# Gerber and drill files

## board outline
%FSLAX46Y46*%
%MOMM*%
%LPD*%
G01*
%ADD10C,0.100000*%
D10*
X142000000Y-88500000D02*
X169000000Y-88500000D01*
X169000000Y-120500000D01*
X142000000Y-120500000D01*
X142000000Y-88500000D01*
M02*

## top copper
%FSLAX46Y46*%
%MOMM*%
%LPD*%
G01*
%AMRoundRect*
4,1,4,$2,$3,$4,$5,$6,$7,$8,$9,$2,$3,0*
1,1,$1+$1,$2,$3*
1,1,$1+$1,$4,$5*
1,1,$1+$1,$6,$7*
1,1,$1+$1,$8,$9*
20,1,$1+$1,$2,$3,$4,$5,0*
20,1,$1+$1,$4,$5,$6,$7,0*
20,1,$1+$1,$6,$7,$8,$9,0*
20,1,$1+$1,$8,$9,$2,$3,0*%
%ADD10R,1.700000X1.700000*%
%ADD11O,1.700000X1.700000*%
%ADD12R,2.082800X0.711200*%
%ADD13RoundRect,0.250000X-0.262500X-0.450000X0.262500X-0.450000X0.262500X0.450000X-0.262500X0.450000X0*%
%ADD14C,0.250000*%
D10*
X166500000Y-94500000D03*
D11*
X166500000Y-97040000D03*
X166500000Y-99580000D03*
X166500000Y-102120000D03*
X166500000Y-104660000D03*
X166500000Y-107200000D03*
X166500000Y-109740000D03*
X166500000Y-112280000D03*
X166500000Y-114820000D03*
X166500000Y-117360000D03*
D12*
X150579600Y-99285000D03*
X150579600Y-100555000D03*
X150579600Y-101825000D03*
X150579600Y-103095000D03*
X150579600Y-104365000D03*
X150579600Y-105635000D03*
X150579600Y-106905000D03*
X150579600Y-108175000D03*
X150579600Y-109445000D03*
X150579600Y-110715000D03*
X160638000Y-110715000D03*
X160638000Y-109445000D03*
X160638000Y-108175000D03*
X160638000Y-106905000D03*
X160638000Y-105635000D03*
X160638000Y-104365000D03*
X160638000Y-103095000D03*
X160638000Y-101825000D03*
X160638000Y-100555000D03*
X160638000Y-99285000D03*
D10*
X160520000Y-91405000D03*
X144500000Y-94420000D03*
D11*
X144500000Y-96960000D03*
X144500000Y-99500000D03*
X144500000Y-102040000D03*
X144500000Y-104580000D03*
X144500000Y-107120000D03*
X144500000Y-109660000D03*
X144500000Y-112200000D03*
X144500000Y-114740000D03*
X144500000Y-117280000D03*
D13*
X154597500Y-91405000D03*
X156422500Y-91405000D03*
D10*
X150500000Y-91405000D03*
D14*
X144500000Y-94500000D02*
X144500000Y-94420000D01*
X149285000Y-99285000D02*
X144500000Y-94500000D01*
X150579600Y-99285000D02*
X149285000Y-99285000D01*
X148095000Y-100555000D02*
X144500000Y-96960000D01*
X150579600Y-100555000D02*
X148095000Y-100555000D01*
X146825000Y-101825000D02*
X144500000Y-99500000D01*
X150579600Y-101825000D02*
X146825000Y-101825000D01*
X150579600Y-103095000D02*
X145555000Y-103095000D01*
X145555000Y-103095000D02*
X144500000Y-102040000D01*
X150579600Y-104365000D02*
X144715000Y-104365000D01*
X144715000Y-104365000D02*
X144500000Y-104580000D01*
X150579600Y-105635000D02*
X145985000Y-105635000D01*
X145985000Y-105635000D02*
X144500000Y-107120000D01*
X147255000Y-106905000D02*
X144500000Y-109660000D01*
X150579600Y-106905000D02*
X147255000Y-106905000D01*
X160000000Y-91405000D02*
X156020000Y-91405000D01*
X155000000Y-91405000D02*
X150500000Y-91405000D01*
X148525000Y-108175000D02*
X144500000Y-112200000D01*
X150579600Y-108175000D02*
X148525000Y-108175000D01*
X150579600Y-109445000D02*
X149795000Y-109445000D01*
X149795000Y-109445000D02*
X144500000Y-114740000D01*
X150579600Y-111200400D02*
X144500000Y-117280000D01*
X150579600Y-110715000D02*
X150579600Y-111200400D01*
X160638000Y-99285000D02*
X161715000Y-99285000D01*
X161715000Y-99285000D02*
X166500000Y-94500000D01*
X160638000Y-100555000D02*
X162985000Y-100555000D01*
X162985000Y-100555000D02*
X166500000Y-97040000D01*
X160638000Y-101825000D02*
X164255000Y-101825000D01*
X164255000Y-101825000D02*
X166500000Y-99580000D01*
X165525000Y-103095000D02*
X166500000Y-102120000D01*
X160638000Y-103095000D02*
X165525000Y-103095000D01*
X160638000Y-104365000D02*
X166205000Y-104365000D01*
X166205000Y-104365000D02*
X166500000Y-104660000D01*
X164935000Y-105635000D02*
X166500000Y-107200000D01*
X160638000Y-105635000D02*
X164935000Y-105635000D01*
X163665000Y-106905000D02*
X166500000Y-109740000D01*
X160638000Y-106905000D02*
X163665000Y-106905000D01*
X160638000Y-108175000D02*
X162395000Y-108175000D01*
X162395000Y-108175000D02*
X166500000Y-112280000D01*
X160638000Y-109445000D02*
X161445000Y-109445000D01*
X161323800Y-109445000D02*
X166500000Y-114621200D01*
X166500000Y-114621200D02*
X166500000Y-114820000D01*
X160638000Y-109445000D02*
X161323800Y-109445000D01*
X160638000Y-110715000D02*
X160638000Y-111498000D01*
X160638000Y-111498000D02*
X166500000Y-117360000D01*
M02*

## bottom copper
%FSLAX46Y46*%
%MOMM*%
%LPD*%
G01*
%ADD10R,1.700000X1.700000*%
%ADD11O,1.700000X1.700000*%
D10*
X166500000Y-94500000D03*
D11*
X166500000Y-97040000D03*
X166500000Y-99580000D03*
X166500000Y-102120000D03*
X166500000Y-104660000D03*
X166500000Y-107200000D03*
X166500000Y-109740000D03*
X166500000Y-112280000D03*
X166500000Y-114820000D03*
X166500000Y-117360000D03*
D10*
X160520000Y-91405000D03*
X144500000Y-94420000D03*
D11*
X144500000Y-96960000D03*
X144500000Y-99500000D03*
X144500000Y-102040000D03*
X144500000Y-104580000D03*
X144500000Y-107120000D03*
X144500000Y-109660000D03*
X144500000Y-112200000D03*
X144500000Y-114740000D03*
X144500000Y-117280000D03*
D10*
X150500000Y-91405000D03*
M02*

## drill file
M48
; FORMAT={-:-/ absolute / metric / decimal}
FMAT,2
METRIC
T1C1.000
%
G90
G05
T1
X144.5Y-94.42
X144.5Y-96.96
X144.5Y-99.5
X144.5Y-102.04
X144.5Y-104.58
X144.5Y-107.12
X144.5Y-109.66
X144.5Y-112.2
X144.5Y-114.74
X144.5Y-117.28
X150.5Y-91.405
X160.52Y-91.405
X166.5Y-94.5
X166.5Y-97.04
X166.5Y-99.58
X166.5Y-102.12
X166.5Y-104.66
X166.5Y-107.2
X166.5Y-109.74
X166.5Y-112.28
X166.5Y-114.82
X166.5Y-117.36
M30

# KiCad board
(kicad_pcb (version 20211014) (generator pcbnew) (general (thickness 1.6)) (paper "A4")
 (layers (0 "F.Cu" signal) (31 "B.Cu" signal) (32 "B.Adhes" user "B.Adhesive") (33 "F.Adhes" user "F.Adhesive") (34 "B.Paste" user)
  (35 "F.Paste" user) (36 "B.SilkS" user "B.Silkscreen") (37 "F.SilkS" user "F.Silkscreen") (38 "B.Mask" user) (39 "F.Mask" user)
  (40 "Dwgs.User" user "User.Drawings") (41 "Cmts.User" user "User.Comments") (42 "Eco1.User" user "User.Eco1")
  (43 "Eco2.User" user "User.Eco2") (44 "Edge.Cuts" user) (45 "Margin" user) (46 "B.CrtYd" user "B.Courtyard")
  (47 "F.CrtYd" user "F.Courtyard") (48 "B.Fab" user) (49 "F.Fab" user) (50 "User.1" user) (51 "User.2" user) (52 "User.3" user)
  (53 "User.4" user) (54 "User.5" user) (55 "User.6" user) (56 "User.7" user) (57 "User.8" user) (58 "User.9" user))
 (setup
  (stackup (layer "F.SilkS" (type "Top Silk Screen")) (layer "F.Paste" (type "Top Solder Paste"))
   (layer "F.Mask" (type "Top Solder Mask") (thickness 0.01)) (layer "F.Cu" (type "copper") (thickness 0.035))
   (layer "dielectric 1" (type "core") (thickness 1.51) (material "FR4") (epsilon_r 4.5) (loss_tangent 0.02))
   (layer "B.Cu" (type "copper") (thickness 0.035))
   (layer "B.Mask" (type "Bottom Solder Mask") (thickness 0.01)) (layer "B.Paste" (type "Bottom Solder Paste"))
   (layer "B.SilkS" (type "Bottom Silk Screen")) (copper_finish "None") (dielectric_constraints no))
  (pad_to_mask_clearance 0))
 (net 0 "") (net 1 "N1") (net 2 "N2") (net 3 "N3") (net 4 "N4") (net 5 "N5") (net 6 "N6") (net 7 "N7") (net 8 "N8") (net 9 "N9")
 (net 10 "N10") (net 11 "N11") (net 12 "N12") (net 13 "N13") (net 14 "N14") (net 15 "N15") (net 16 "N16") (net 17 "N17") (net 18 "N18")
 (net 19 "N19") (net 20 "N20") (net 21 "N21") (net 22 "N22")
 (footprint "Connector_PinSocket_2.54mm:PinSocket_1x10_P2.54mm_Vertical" (layer "F.Cu") (at 166.5 94.5)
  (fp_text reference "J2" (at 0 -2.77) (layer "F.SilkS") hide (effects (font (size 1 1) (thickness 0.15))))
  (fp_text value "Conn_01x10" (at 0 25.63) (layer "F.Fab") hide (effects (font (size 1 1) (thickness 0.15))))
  (pad "1" thru_hole rect (at 0 0) (size 1.7 1.7) (drill 1) (layers *.Cu *.Mask) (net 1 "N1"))
  (pad "2" thru_hole oval (at 0 2.54) (size 1.7 1.7) (drill 1) (layers *.Cu *.Mask) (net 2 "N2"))
  (pad "3" thru_hole oval (at 0 5.08) (size 1.7 1.7) (drill 1) (layers *.Cu *.Mask) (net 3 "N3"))
  (pad "4" thru_hole oval (at 0 7.62) (size 1.7 1.7) (drill 1) (layers *.Cu *.Mask) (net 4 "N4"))
  (pad "5" thru_hole oval (at 0 10.16) (size 1.7 1.7) (drill 1) (layers *.Cu *.Mask) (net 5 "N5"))
  (pad "6" thru_hole oval (at 0 12.7) (size 1.7 1.7) (drill 1) (layers *.Cu *.Mask) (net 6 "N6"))
  (pad "7" thru_hole oval (at 0 15.24) (size 1.7 1.7) (drill 1) (layers *.Cu *.Mask) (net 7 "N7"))
  (pad "8" thru_hole oval (at 0 17.78) (size 1.7 1.7) (drill 1) (layers *.Cu *.Mask) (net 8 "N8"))
  (pad "9" thru_hole oval (at 0 20.32) (size 1.7 1.7) (drill 1) (layers *.Cu *.Mask) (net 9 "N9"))
  (pad "10" thru_hole oval (at 0 22.86) (size 1.7 1.7) (drill 1) (layers *.Cu *.Mask) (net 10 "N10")))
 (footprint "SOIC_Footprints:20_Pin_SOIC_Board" (layer "F.Cu") (at 156.32 105)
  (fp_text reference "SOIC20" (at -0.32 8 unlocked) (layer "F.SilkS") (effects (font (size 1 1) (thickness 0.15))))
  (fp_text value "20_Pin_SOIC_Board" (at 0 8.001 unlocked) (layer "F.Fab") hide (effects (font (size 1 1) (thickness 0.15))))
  (pad "1" smd rect (at -5.7404 -5.715) (size 2.0828 0.7112) (layers "F.Cu" "F.Paste" "F.Mask") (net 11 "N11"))
  (pad "2" smd rect (at -5.7404 -4.445) (size 2.0828 0.7112) (layers "F.Cu" "F.Paste" "F.Mask") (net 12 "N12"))
  (pad "3" smd rect (at -5.7404 -3.175) (size 2.0828 0.7112) (layers "F.Cu" "F.Paste" "F.Mask") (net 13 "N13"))
  (pad "4" smd rect (at -5.7404 -1.905) (size 2.0828 0.7112) (layers "F.Cu" "F.Paste" "F.Mask") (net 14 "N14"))
  (pad "5" smd rect (at -5.7404 -0.635) (size 2.0828 0.7112) (layers "F.Cu" "F.Paste" "F.Mask") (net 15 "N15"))
  (pad "6" smd rect (at -5.7404 0.635) (size 2.0828 0.7112) (layers "F.Cu" "F.Paste" "F.Mask") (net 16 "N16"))
  (pad "7" smd rect (at -5.7404 1.905) (size 2.0828 0.7112) (layers "F.Cu" "F.Paste" "F.Mask") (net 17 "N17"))
  (pad "8" smd rect (at -5.7404 3.175) (size 2.0828 0.7112) (layers "F.Cu" "F.Paste" "F.Mask") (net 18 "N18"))
  (pad "9" smd rect (at -5.7404 4.445) (size 2.0828 0.7112) (layers "F.Cu" "F.Paste" "F.Mask") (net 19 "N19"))
  (pad "10" smd rect (at -5.7404 5.715) (size 2.0828 0.7112) (layers "F.Cu" "F.Paste" "F.Mask") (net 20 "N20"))
  (pad "11" smd rect (at 4.318 5.715) (size 2.0828 0.7112) (layers "F.Cu" "F.Paste" "F.Mask") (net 10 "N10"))
  (pad "12" smd rect (at 4.318 4.445) (size 2.0828 0.7112) (layers "F.Cu" "F.Paste" "F.Mask") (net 9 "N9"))
  (pad "13" smd rect (at 4.318 3.175) (size 2.0828 0.7112) (layers "F.Cu" "F.Paste" "F.Mask") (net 8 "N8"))
  (pad "14" smd rect (at 4.318 1.905) (size 2.0828 0.7112) (layers "F.Cu" "F.Paste" "F.Mask") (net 7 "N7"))
  (pad "15" smd rect (at 4.318 0.635) (size 2.0828 0.7112) (layers "F.Cu" "F.Paste" "F.Mask") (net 6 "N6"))
  (pad "16" smd rect (at 4.318 -0.635) (size 2.0828 0.7112) (layers "F.Cu" "F.Paste" "F.Mask") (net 5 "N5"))
  (pad "17" smd rect (at 4.318 -1.905) (size 2.0828 0.7112) (layers "F.Cu" "F.Paste" "F.Mask") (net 4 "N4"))
  (pad "18" smd rect (at 4.318 -3.175) (size 2.0828 0.7112) (layers "F.Cu" "F.Paste" "F.Mask") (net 3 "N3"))
  (pad "19" smd rect (at 4.318 -4.445) (size 2.0828 0.7112) (layers "F.Cu" "F.Paste" "F.Mask") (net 2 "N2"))
  (pad "20" smd rect (at 4.318 -5.715) (size 2.0828 0.7112) (layers "F.Cu" "F.Paste" "F.Mask") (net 1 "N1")))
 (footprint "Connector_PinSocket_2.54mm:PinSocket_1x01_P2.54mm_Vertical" (layer "F.Cu") (at 160.52 91.405)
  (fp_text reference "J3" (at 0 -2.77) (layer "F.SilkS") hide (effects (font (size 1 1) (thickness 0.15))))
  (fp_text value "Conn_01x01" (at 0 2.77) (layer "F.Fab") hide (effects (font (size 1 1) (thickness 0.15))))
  (pad "1" thru_hole rect (at 0 0) (size 1.7 1.7) (drill 1) (layers *.Cu *.Mask) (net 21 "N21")))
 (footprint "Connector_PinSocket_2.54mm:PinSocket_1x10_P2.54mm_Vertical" (layer "F.Cu") (at 144.5 94.42)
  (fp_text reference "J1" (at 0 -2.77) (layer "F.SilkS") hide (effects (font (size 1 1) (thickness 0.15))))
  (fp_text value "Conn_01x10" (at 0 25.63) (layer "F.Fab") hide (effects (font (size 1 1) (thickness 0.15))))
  (pad "1" thru_hole rect (at 0 0) (size 1.7 1.7) (drill 1) (layers *.Cu *.Mask) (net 11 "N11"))
  (pad "2" thru_hole oval (at 0 2.54) (size 1.7 1.7) (drill 1) (layers *.Cu *.Mask) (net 12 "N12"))
  (pad "3" thru_hole oval (at 0 5.08) (size 1.7 1.7) (drill 1) (layers *.Cu *.Mask) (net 13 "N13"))
  (pad "4" thru_hole oval (at 0 7.62) (size 1.7 1.7) (drill 1) (layers *.Cu *.Mask) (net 14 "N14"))
  (pad "5" thru_hole oval (at 0 10.16) (size 1.7 1.7) (drill 1) (layers *.Cu *.Mask) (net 15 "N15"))
  (pad "6" thru_hole oval (at 0 12.7) (size 1.7 1.7) (drill 1) (layers *.Cu *.Mask) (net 16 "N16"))
  (pad "7" thru_hole oval (at 0 15.24) (size 1.7 1.7) (drill 1) (layers *.Cu *.Mask) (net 17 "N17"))
  (pad "8" thru_hole oval (at 0 17.78) (size 1.7 1.7) (drill 1) (layers *.Cu *.Mask) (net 18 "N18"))
  (pad "9" thru_hole oval (at 0 20.32) (size 1.7 1.7) (drill 1) (layers *.Cu *.Mask) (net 19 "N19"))
  (pad "10" thru_hole oval (at 0 22.86) (size 1.7 1.7) (drill 1) (layers *.Cu *.Mask) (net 20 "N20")))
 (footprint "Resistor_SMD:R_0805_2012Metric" (layer "F.Cu") (at 155.51 91.405)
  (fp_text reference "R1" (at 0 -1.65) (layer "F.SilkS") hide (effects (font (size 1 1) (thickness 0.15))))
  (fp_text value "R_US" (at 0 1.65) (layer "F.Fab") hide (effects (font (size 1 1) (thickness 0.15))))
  (pad "1" smd roundrect (at -0.9125 0) (size 1.025 1.4) (layers "F.Cu" "F.Paste" "F.Mask") (roundrect_rratio 0.243902) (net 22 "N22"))
  (pad "2" smd roundrect (at 0.9125 0) (size 1.025 1.4) (layers "F.Cu" "F.Paste" "F.Mask") (roundrect_rratio 0.243902) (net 21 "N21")))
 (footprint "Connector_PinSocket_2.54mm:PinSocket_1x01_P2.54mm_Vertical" (layer "F.Cu") (at 150.5 91.405)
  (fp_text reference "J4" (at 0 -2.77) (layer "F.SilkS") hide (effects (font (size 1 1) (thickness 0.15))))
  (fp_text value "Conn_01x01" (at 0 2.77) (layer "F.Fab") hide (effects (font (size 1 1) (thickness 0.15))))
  (pad "1" thru_hole rect (at 0 0) (size 1.7 1.7) (drill 1) (layers *.Cu *.Mask) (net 22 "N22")))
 (gr_rect (start 142 88.5) (end 169 120.5) (layer "Edge.Cuts") (width 0.1) (fill none))
 (segment (start 144.5 94.5) (end 144.5 94.42) (width 0.25) (layer "F.Cu") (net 11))
 (segment (start 149.285 99.285) (end 144.5 94.5) (width 0.25) (layer "F.Cu") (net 11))
 (segment (start 150.5796 99.285) (end 149.285 99.285) (width 0.25) (layer "F.Cu") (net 11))
 (segment (start 148.095 100.555) (end 144.5 96.96) (width 0.25) (layer "F.Cu") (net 12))
 (segment (start 150.5796 100.555) (end 148.095 100.555) (width 0.25) (layer "F.Cu") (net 12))
 (segment (start 146.825 101.825) (end 144.5 99.5) (width 0.25) (layer "F.Cu") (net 13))
 (segment (start 150.5796 101.825) (end 146.825 101.825) (width 0.25) (layer "F.Cu") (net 13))
 (segment (start 150.5796 103.095) (end 145.555 103.095) (width 0.25) (layer "F.Cu") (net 14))
 (segment (start 145.555 103.095) (end 144.5 102.04) (width 0.25) (layer "F.Cu") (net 14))
 (segment (start 150.5796 104.365) (end 144.715 104.365) (width 0.25) (layer "F.Cu") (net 15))
 (segment (start 144.715 104.365) (end 144.5 104.58) (width 0.25) (layer "F.Cu") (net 15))
 (segment (start 150.5796 105.635) (end 145.985 105.635) (width 0.25) (layer "F.Cu") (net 16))
 (segment (start 145.985 105.635) (end 144.5 107.12) (width 0.25) (layer "F.Cu") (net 16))
 (segment (start 147.255 106.905) (end 144.5 109.66) (width 0.25) (layer "F.Cu") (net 17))
 (segment (start 150.5796 106.905) (end 147.255 106.905) (width 0.25) (layer "F.Cu") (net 17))
 (segment (start 160 91.405) (end 156.02 91.405) (width 0.25) (layer "F.Cu") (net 21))
 (segment (start 155 91.405) (end 150.5 91.405) (width 0.25) (layer "F.Cu") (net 22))
 (segment (start 148.525 108.175) (end 144.5 112.2) (width 0.25) (layer "F.Cu") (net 18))
 (segment (start 150.5796 108.175) (end 148.525 108.175) (width 0.25) (layer "F.Cu") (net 18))
 (segment (start 150.5796 109.445) (end 149.795 109.445) (width 0.25) (layer "F.Cu") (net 19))
 (segment (start 149.795 109.445) (end 144.5 114.74) (width 0.25) (layer "F.Cu") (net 19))
 (segment (start 150.5796 111.2004) (end 144.5 117.28) (width 0.25) (layer "F.Cu") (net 20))
 (segment (start 150.5796 110.715) (end 150.5796 111.2004) (width 0.25) (layer "F.Cu") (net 20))
 (segment (start 160.638 99.285) (end 161.715 99.285) (width 0.25) (layer "F.Cu") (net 1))
 (segment (start 161.715 99.285) (end 166.5 94.5) (width 0.25) (layer "F.Cu") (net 1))
 (segment (start 160.638 100.555) (end 162.985 100.555) (width 0.25) (layer "F.Cu") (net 2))
 (segment (start 162.985 100.555) (end 166.5 97.04) (width 0.25) (layer "F.Cu") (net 2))
 (segment (start 160.638 101.825) (end 164.255 101.825) (width 0.25) (layer "F.Cu") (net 3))
 (segment (start 164.255 101.825) (end 166.5 99.58) (width 0.25) (layer "F.Cu") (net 3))
 (segment (start 165.525 103.095) (end 166.5 102.12) (width 0.25) (layer "F.Cu") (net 4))
 (segment (start 160.638 103.095) (end 165.525 103.095) (width 0.25) (layer "F.Cu") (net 4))
 (segment (start 160.638 104.365) (end 166.205 104.365) (width 0.25) (layer "F.Cu") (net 5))
 (segment (start 166.205 104.365) (end 166.5 104.66) (width 0.25) (layer "F.Cu") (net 5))
 (segment (start 164.935 105.635) (end 166.5 107.2) (width 0.25) (layer "F.Cu") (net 6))
 (segment (start 160.638 105.635) (end 164.935 105.635) (width 0.25) (layer "F.Cu") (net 6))
 (segment (start 163.665 106.905) (end 166.5 109.74) (width 0.25) (layer "F.Cu") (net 7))
 (segment (start 160.638 106.905) (end 163.665 106.905) (width 0.25) (layer "F.Cu") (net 7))
 (segment (start 160.638 108.175) (end 162.395 108.175) (width 0.25) (layer "F.Cu") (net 8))
 (segment (start 162.395 108.175) (end 166.5 112.28) (width 0.25) (layer "F.Cu") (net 8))
 (segment (start 160.638 109.445) (end 161.445 109.445) (width 0.25) (layer "F.Cu") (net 9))
 (segment (start 161.3238 109.445) (end 166.5 114.6212) (width 0.25) (layer "F.Cu") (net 9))
 (segment (start 166.5 114.6212) (end 166.5 114.82) (width 0.25) (layer "F.Cu") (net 9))
 (segment (start 160.638 109.445) (end 161.3238 109.445) (width 0.25) (layer "F.Cu") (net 9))
 (segment (start 160.638 110.715) (end 160.638 111.498) (width 0.25) (layer "F.Cu") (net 10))
 (segment (start 160.638 111.498) (end 166.5 117.36) (width 0.25) (layer "F.Cu") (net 10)))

